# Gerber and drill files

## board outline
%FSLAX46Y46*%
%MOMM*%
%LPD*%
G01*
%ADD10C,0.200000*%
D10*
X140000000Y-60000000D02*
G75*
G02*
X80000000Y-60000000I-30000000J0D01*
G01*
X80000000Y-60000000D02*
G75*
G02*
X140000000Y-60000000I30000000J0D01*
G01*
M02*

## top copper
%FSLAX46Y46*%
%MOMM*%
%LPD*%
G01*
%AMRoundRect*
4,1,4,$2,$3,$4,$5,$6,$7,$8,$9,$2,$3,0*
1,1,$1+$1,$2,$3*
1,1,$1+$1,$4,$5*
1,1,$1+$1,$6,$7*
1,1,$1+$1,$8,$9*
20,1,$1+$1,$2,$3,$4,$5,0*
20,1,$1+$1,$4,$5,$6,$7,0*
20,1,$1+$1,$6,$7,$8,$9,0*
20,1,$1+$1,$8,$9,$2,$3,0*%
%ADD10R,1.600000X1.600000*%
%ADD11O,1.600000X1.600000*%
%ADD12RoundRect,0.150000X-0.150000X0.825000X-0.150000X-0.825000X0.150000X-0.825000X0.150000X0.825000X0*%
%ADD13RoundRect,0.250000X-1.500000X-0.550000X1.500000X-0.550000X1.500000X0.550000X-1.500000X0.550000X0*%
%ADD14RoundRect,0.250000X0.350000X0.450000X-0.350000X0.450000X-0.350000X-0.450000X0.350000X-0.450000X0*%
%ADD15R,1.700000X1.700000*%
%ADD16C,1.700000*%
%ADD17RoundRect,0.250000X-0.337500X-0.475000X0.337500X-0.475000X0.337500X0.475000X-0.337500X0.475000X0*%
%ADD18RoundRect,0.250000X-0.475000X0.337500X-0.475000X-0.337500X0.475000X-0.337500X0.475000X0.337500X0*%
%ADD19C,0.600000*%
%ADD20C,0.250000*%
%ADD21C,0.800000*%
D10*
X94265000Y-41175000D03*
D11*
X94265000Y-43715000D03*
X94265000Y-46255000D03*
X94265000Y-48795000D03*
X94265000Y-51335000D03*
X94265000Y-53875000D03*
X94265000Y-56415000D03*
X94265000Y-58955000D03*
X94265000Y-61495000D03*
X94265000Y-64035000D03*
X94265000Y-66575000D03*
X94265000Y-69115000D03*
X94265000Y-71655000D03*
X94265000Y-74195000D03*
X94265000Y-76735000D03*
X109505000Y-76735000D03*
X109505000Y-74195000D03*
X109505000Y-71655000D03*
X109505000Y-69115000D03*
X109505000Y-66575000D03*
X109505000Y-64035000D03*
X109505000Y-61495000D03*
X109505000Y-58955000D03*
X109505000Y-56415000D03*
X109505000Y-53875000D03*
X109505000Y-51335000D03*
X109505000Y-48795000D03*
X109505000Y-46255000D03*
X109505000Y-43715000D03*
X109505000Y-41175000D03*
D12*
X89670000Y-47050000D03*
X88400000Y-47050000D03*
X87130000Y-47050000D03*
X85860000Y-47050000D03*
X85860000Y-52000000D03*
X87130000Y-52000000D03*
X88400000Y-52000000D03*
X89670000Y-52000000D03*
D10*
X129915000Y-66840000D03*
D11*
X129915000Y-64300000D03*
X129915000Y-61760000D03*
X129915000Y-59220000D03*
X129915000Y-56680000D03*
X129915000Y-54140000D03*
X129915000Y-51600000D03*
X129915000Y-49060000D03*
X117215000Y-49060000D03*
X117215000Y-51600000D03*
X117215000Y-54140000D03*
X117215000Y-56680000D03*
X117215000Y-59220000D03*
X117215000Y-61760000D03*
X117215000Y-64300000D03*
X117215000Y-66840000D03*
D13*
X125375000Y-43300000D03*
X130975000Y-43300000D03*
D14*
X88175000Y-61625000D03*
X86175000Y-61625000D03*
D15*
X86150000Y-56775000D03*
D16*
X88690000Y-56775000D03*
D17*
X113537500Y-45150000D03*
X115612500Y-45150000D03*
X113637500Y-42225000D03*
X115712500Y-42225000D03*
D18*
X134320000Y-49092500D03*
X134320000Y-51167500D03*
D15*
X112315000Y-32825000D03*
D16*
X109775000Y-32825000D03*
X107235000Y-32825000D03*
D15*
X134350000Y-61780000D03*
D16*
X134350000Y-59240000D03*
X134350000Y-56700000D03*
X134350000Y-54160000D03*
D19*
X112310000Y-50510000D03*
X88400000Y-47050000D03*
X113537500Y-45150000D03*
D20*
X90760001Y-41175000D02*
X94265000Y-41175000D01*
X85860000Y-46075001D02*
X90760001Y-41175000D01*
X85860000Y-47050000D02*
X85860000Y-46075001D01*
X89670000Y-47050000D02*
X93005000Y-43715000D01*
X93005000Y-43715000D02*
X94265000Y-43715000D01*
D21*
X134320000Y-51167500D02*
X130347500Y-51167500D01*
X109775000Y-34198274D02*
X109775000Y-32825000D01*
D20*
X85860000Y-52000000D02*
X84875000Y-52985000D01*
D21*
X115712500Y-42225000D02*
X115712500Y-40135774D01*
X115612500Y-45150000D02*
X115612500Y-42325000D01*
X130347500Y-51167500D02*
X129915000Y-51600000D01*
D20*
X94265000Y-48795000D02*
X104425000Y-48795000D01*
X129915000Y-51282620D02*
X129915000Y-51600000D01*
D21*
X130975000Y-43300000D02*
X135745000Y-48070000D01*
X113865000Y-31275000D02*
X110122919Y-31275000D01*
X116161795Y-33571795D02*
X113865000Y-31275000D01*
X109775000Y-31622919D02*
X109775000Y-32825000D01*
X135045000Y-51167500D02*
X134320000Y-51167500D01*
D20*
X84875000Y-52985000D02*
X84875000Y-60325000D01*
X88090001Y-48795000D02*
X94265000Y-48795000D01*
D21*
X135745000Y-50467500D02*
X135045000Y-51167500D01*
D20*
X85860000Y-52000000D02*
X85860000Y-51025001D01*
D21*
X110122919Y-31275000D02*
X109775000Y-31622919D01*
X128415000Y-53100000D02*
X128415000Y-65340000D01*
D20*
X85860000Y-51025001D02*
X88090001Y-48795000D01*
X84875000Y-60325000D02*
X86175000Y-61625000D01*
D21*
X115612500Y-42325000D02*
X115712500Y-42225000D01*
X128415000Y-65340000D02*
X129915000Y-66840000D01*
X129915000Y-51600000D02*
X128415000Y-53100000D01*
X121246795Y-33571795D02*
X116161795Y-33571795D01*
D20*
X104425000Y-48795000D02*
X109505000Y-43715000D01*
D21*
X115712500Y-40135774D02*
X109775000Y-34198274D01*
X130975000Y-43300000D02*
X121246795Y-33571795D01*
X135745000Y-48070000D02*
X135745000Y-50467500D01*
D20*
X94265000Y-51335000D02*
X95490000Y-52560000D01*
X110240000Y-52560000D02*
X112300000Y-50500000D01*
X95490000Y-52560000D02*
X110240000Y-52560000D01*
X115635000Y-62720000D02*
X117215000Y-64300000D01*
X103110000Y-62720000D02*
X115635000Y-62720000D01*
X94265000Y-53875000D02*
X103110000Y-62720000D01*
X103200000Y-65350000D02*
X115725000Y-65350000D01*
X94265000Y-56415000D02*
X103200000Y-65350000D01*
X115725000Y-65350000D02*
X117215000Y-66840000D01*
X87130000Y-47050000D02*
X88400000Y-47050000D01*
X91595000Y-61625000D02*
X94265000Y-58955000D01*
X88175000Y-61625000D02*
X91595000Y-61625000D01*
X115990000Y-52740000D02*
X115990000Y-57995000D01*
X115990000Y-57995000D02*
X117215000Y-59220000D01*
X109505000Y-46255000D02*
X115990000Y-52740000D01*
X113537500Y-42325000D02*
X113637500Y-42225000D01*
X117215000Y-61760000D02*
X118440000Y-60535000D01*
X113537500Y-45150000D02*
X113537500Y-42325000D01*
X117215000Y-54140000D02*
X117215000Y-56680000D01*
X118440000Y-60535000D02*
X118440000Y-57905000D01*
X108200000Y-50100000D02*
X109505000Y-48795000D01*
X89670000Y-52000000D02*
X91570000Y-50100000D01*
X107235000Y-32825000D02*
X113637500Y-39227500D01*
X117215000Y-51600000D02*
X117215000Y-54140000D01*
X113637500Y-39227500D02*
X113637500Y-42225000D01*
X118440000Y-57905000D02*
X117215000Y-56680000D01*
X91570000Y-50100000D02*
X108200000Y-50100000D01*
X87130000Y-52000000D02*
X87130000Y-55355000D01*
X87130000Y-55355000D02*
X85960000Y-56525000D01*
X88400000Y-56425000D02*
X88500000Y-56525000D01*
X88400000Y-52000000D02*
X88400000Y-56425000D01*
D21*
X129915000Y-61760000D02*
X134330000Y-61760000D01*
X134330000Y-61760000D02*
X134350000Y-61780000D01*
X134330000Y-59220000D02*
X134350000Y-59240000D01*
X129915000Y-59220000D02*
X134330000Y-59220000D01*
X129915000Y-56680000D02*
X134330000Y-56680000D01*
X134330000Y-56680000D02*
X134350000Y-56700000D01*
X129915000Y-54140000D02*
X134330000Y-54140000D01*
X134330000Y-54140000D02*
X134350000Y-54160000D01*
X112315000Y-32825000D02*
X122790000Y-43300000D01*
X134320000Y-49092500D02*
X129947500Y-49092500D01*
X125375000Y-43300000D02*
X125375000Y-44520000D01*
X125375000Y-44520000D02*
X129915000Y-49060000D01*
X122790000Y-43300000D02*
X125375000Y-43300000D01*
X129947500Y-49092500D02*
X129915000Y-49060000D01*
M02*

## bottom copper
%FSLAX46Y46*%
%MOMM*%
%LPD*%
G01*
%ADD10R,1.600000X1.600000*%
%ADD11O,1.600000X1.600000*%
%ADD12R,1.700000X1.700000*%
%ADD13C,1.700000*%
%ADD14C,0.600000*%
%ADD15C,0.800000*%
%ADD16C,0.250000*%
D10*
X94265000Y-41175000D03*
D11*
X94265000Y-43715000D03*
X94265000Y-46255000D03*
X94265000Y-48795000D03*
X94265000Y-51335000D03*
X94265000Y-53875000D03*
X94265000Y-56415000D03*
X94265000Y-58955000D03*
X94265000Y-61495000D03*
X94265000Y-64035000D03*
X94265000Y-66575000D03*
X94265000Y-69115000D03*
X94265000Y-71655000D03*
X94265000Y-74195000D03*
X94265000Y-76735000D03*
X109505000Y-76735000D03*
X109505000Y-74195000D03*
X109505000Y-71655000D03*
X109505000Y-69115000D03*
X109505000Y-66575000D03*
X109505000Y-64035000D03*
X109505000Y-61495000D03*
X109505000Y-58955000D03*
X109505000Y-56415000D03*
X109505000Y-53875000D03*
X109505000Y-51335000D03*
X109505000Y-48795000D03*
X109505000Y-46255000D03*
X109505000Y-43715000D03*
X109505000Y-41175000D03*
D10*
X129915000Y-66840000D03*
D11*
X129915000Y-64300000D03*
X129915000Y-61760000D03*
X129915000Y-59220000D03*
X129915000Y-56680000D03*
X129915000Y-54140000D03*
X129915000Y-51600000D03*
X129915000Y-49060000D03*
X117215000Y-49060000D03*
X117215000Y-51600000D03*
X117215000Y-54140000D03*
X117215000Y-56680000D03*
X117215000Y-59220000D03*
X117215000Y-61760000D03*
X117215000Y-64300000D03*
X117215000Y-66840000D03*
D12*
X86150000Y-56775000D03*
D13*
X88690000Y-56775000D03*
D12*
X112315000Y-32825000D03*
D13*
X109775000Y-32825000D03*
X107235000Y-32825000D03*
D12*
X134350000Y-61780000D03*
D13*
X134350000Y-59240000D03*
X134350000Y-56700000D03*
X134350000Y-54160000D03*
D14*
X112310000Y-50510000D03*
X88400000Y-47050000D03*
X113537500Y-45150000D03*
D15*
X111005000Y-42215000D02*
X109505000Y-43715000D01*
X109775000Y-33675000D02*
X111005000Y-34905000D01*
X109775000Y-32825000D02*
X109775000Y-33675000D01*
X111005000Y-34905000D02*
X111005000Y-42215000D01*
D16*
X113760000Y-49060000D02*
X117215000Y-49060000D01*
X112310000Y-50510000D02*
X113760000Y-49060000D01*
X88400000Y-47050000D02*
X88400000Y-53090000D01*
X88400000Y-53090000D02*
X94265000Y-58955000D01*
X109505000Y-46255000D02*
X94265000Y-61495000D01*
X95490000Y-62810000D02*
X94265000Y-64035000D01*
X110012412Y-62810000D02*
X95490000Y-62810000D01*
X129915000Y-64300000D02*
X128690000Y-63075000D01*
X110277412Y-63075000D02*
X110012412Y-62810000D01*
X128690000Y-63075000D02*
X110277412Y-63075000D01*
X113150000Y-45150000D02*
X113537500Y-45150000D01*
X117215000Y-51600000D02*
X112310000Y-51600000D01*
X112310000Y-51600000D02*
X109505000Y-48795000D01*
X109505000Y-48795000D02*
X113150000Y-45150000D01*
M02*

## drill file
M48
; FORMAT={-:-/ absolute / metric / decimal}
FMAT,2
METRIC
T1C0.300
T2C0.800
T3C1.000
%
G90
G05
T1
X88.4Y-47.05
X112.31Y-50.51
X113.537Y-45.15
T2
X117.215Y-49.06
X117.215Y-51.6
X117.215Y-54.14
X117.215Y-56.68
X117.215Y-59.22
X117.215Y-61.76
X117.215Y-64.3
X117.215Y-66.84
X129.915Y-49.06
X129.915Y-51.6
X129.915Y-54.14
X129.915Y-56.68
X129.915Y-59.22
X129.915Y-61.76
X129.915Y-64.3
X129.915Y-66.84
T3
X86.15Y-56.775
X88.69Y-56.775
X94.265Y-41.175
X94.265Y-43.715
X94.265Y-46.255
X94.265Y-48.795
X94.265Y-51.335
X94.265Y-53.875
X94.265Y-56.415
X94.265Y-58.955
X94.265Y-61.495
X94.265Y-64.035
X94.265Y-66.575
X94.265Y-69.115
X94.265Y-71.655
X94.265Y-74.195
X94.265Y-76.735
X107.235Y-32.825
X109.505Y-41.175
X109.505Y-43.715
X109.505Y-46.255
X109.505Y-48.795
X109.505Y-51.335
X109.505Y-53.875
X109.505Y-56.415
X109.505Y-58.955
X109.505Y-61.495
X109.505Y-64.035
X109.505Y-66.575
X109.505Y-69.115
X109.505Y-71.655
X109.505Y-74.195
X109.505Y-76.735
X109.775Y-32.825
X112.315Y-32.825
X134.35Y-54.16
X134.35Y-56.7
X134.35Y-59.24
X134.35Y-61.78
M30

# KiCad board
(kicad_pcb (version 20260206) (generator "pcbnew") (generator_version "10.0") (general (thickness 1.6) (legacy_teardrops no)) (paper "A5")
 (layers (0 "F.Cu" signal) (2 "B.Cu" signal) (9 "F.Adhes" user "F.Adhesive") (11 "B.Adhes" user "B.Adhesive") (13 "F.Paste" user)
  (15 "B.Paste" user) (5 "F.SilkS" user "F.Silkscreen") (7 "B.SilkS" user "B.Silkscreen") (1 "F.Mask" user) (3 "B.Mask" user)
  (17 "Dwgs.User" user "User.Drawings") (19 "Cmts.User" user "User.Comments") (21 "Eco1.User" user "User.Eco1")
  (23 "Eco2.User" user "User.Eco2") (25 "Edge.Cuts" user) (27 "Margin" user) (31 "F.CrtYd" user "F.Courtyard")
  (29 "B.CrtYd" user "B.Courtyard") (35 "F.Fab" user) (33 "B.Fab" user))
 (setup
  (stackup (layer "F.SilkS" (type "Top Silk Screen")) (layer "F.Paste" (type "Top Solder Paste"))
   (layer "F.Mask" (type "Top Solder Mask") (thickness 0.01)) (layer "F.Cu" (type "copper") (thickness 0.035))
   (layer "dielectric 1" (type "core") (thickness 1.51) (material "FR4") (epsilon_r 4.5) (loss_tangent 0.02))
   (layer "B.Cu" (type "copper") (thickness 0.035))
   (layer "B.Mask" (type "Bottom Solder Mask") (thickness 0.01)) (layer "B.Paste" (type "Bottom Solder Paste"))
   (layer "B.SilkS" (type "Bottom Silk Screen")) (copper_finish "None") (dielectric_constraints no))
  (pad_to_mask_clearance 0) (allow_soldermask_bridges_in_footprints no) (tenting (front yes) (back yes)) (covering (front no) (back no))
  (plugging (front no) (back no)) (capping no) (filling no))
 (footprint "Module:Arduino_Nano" (layer "F.Cu") (at 94.265 41.175)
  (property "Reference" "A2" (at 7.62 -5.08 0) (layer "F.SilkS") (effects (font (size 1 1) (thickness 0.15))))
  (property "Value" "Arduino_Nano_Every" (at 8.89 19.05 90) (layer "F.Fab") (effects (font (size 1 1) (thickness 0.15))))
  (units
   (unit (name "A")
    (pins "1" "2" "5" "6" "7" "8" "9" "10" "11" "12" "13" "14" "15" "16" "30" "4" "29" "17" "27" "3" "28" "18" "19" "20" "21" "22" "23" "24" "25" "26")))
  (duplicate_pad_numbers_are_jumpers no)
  (pad "1" thru_hole rect (at 0 0) (size 1.6 1.6) (drill 1) (layers "*.Cu" "*.Mask") (remove_unused_layers no) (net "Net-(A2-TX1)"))
  (pad "2" thru_hole oval (at 0 2.54) (size 1.6 1.6) (drill 1) (layers "*.Cu" "*.Mask") (remove_unused_layers no) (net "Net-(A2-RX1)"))
  (pad "3" thru_hole oval (at 0 5.08) (size 1.6 1.6) (drill 1) (layers "*.Cu" "*.Mask") (remove_unused_layers no)
   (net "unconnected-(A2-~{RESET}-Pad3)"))
  (pad "4" thru_hole oval (at 0 7.62) (size 1.6 1.6) (drill 1) (layers "*.Cu" "*.Mask") (remove_unused_layers no) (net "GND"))
  (pad "5" thru_hole oval (at 0 10.16) (size 1.6 1.6) (drill 1) (layers "*.Cu" "*.Mask") (remove_unused_layers no) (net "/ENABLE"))
  (pad "6" thru_hole oval (at 0 12.7) (size 1.6 1.6) (drill 1) (layers "*.Cu" "*.Mask") (remove_unused_layers no) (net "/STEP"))
  (pad "7" thru_hole oval (at 0 15.24) (size 1.6 1.6) (drill 1) (layers "*.Cu" "*.Mask") (remove_unused_layers no) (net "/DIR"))
  (pad "8" thru_hole oval (at 0 17.78) (size 1.6 1.6) (drill 1) (layers "*.Cu" "*.Mask") (remove_unused_layers no) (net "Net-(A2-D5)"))
  (pad "9" thru_hole oval (at 0 20.32) (size 1.6 1.6) (drill 1) (layers "*.Cu" "*.Mask") (remove_unused_layers no) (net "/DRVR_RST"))
  (pad "10" thru_hole oval (at 0 22.86) (size 1.6 1.6) (drill 1) (layers "*.Cu" "*.Mask") (remove_unused_layers no) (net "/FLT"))
  (pad "11" thru_hole oval (at 0 25.4) (size 1.6 1.6) (drill 1) (layers "*.Cu" "*.Mask") (remove_unused_layers no)
   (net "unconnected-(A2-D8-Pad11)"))
  (pad "12" thru_hole oval (at 0 27.94) (size 1.6 1.6) (drill 1) (layers "*.Cu" "*.Mask") (remove_unused_layers no)
   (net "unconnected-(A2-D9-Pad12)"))
  (pad "13" thru_hole oval (at 0 30.48) (size 1.6 1.6) (drill 1) (layers "*.Cu" "*.Mask") (remove_unused_layers no)
   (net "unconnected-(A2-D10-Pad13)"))
  (pad "14" thru_hole oval (at 0 33.02) (size 1.6 1.6) (drill 1) (layers "*.Cu" "*.Mask") (remove_unused_layers no)
   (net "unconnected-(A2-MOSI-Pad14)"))
  (pad "15" thru_hole oval (at 0 35.56) (size 1.6 1.6) (drill 1) (layers "*.Cu" "*.Mask") (remove_unused_layers no)
   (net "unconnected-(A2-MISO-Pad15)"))
  (pad "16" thru_hole oval (at 15.24 35.56) (size 1.6 1.6) (drill 1) (layers "*.Cu" "*.Mask") (remove_unused_layers no)
   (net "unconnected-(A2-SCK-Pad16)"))
  (pad "17" thru_hole oval (at 15.24 33.02) (size 1.6 1.6) (drill 1) (layers "*.Cu" "*.Mask") (remove_unused_layers no)
   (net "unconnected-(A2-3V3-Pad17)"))
  (pad "18" thru_hole oval (at 15.24 30.48) (size 1.6 1.6) (drill 1) (layers "*.Cu" "*.Mask") (remove_unused_layers no)
   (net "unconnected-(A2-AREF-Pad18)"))
  (pad "19" thru_hole oval (at 15.24 27.94) (size 1.6 1.6) (drill 1) (layers "*.Cu" "*.Mask") (remove_unused_layers no)
   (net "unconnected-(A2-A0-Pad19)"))
  (pad "20" thru_hole oval (at 15.24 25.4) (size 1.6 1.6) (drill 1) (layers "*.Cu" "*.Mask") (remove_unused_layers no)
   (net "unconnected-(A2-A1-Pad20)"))
  (pad "21" thru_hole oval (at 15.24 22.86) (size 1.6 1.6) (drill 1) (layers "*.Cu" "*.Mask") (remove_unused_layers no)
   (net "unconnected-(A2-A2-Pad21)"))
  (pad "22" thru_hole oval (at 15.24 20.32) (size 1.6 1.6) (drill 1) (layers "*.Cu" "*.Mask") (remove_unused_layers no)
   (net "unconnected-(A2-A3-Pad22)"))
  (pad "23" thru_hole oval (at 15.24 17.78) (size 1.6 1.6) (drill 1) (layers "*.Cu" "*.Mask") (remove_unused_layers no)
   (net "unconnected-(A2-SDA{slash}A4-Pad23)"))
  (pad "24" thru_hole oval (at 15.24 15.24) (size 1.6 1.6) (drill 1) (layers "*.Cu" "*.Mask") (remove_unused_layers no)
   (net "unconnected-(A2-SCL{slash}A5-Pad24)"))
  (pad "25" thru_hole oval (at 15.24 12.7) (size 1.6 1.6) (drill 1) (layers "*.Cu" "*.Mask") (remove_unused_layers no)
   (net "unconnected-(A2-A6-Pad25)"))
  (pad "26" thru_hole oval (at 15.24 10.16) (size 1.6 1.6) (drill 1) (layers "*.Cu" "*.Mask") (remove_unused_layers no)
   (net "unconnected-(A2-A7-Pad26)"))
  (pad "27" thru_hole oval (at 15.24 7.62) (size 1.6 1.6) (drill 1) (layers "*.Cu" "*.Mask") (remove_unused_layers no) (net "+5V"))
  (pad "28" thru_hole oval (at 15.24 5.08) (size 1.6 1.6) (drill 1) (layers "*.Cu" "*.Mask") (remove_unused_layers no) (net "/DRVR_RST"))
  (pad "29" thru_hole oval (at 15.24 2.54) (size 1.6 1.6) (drill 1) (layers "*.Cu" "*.Mask") (remove_unused_layers no) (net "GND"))
  (pad "30" thru_hole oval (at 15.24 0) (size 1.6 1.6) (drill 1) (layers "*.Cu" "*.Mask") (remove_unused_layers no)
   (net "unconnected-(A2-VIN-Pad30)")))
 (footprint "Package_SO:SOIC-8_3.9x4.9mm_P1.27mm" (layer "F.Cu") (at 87.765 49.525 -90)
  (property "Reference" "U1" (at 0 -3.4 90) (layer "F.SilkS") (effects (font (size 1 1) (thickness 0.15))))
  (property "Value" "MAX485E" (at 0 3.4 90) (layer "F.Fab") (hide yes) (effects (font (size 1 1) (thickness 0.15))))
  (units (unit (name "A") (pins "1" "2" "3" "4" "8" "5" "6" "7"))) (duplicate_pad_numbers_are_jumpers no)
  (pad "1" smd roundrect (at -2.475 -1.905 270) (size 1.95 0.6) (layers "F.Cu" "F.Mask" "F.Paste") (roundrect_rratio 0.25)
   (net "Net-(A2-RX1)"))
  (pad "2" smd roundrect (at -2.475 -0.635 270) (size 1.95 0.6) (layers "F.Cu" "F.Mask" "F.Paste") (roundrect_rratio 0.25)
   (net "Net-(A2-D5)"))
  (pad "3" smd roundrect (at -2.475 0.635 270) (size 1.95 0.6) (layers "F.Cu" "F.Mask" "F.Paste") (roundrect_rratio 0.25)
   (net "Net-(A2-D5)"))
  (pad "4" smd roundrect (at -2.475 1.905 270) (size 1.95 0.6) (layers "F.Cu" "F.Mask" "F.Paste") (roundrect_rratio 0.25)
   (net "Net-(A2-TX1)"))
  (pad "5" smd roundrect (at 2.475 1.905 270) (size 1.95 0.6) (layers "F.Cu" "F.Mask" "F.Paste") (roundrect_rratio 0.25) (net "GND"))
  (pad "6" smd roundrect (at 2.475 0.635 270) (size 1.95 0.6) (layers "F.Cu" "F.Mask" "F.Paste") (roundrect_rratio 0.25)
   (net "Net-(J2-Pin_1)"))
  (pad "7" smd roundrect (at 2.475 -0.635 270) (size 1.95 0.6) (layers "F.Cu" "F.Mask" "F.Paste") (roundrect_rratio 0.25)
   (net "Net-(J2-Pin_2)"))
  (pad "8" smd roundrect (at 2.475 -1.905 270) (size 1.95 0.6) (layers "F.Cu" "F.Mask" "F.Paste") (roundrect_rratio 0.25) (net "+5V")))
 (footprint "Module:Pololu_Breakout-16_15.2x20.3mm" (layer "F.Cu") (at 129.915 66.84 180)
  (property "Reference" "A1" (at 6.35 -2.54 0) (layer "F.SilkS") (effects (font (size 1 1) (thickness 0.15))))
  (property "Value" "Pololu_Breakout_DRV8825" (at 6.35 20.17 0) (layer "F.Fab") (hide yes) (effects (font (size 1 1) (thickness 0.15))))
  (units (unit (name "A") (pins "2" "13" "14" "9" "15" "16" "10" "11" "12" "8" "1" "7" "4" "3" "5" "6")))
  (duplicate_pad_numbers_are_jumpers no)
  (pad "1" thru_hole rect (at 0 0 180) (size 1.6 1.6) (drill 0.8) (layers "*.Cu" "*.Mask") (remove_unused_layers no) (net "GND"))
  (pad "2" thru_hole oval (at 0 2.54 180) (size 1.6 1.6) (drill 0.8) (layers "*.Cu" "*.Mask") (remove_unused_layers no) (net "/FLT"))
  (pad "3" thru_hole oval (at 0 5.08 180) (size 1.6 1.6) (drill 0.8) (layers "*.Cu" "*.Mask") (remove_unused_layers no) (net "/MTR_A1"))
  (pad "4" thru_hole oval (at 0 7.62 180) (size 1.6 1.6) (drill 0.8) (layers "*.Cu" "*.Mask") (remove_unused_layers no) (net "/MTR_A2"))
  (pad "5" thru_hole oval (at 0 10.16 180) (size 1.6 1.6) (drill 0.8) (layers "*.Cu" "*.Mask") (remove_unused_layers no) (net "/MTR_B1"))
  (pad "6" thru_hole oval (at 0 12.7 180) (size 1.6 1.6) (drill 0.8) (layers "*.Cu" "*.Mask") (remove_unused_layers no) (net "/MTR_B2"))
  (pad "7" thru_hole oval (at 0 15.24 180) (size 1.6 1.6) (drill 0.8) (layers "*.Cu" "*.Mask") (remove_unused_layers no) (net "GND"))
  (pad "8" thru_hole oval (at 0 17.78 180) (size 1.6 1.6) (drill 0.8) (layers "*.Cu" "*.Mask") (remove_unused_layers no) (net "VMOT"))
  (pad "9" thru_hole oval (at 12.7 17.78 180) (size 1.6 1.6) (drill 0.8) (layers "*.Cu" "*.Mask") (remove_unused_layers no) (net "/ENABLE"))
  (pad "10" thru_hole oval (at 12.7 15.24 180) (size 1.6 1.6) (drill 0.8) (layers "*.Cu" "*.Mask") (remove_unused_layers no) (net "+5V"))
  (pad "11" thru_hole oval (at 12.7 12.7 180) (size 1.6 1.6) (drill 0.8) (layers "*.Cu" "*.Mask") (remove_unused_layers no) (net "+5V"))
  (pad "12" thru_hole oval (at 12.7 10.16 180) (size 1.6 1.6) (drill 0.8) (layers "*.Cu" "*.Mask") (remove_unused_layers no) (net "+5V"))
  (pad "13" thru_hole oval (at 12.7 7.62 180) (size 1.6 1.6) (drill 0.8) (layers "*.Cu" "*.Mask") (remove_unused_layers no)
   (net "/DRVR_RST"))
  (pad "14" thru_hole oval (at 12.7 5.08 180) (size 1.6 1.6) (drill 0.8) (layers "*.Cu" "*.Mask") (remove_unused_layers no) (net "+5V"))
  (pad "15" thru_hole oval (at 12.7 2.54 180) (size 1.6 1.6) (drill 0.8) (layers "*.Cu" "*.Mask") (remove_unused_layers no) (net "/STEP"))
  (pad "16" thru_hole oval (at 12.7 0 180) (size 1.6 1.6) (drill 0.8) (layers "*.Cu" "*.Mask") (remove_unused_layers no) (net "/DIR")))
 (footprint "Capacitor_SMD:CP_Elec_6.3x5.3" (layer "F.Cu") (at 128.175 43.3)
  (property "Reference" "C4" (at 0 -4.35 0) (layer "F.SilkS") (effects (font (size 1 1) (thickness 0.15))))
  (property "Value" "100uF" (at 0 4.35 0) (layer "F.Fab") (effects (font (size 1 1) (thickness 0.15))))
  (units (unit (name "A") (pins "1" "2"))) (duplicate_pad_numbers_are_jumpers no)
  (pad "1" smd roundrect (at -2.8 0) (size 3.5 1.6) (layers "F.Cu" "F.Mask" "F.Paste") (roundrect_rratio 0.15625) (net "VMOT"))
  (pad "2" smd roundrect (at 2.8 0) (size 3.5 1.6) (layers "F.Cu" "F.Mask" "F.Paste") (roundrect_rratio 0.15625) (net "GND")))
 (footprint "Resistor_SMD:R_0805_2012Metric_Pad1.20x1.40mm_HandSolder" (layer "F.Cu") (at 87.175 61.625 180)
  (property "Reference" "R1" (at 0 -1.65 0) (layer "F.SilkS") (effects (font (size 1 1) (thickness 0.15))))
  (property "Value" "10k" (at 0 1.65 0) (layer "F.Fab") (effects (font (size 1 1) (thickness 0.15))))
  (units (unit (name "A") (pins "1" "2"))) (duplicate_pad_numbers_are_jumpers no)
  (pad "1" smd roundrect (at -1 0 180) (size 1.2 1.4) (layers "F.Cu" "F.Mask" "F.Paste") (roundrect_rratio 0.208333) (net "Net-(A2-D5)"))
  (pad "2" smd roundrect (at 1 0 180) (size 1.2 1.4) (layers "F.Cu" "F.Mask" "F.Paste") (roundrect_rratio 0.208333) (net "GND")))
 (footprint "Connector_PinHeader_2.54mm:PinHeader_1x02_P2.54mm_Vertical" (layer "F.Cu") (at 86.15 56.775 90)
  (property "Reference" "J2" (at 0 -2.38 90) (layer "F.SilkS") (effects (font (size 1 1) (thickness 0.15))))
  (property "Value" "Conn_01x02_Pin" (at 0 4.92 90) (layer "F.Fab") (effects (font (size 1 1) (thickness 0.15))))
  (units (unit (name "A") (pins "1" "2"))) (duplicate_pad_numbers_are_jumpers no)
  (pad "1" thru_hole rect (at 0 0 90) (size 1.7 1.7) (drill 1) (layers "*.Cu" "*.Mask") (remove_unused_layers no) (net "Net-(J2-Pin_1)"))
  (pad "2" thru_hole circle (at 0 2.54 90) (size 1.7 1.7) (drill 1) (layers "*.Cu" "*.Mask") (remove_unused_layers no)
   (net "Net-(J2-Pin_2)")))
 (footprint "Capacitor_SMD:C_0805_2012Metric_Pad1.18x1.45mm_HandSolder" (layer "F.Cu") (at 114.575 45.15)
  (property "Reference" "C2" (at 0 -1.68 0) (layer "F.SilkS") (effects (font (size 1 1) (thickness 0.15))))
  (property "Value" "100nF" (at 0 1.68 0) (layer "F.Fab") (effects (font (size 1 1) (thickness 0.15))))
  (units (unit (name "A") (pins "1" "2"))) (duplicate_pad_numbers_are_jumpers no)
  (pad "1" smd roundrect (at -1.0375 0) (size 1.175 1.45) (layers "F.Cu" "F.Mask" "F.Paste") (roundrect_rratio 0.212766) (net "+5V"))
  (pad "2" smd roundrect (at 1.0375 0) (size 1.175 1.45) (layers "F.Cu" "F.Mask" "F.Paste") (roundrect_rratio 0.212766) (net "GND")))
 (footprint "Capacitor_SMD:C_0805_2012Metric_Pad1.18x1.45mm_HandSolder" (layer "F.Cu") (at 114.675 42.225)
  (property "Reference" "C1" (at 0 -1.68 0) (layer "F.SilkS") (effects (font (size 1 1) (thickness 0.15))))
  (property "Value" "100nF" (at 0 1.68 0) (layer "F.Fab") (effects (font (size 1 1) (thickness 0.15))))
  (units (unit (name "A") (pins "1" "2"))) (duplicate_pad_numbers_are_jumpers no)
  (pad "1" smd roundrect (at -1.0375 0) (size 1.175 1.45) (layers "F.Cu" "F.Mask" "F.Paste") (roundrect_rratio 0.212766) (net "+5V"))
  (pad "2" smd roundrect (at 1.0375 0) (size 1.175 1.45) (layers "F.Cu" "F.Mask" "F.Paste") (roundrect_rratio 0.212766) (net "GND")))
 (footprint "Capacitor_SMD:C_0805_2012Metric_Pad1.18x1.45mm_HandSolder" (layer "F.Cu") (at 134.32 50.13 -90)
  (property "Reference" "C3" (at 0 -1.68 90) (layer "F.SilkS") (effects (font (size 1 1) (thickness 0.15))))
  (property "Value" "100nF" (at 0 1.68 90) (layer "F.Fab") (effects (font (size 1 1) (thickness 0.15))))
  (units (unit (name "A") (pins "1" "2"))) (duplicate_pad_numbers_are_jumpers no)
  (pad "1" smd roundrect (at -1.0375 0 270) (size 1.175 1.45) (layers "F.Cu" "F.Mask" "F.Paste") (roundrect_rratio 0.212766) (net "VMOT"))
  (pad "2" smd roundrect (at 1.0375 0 270) (size 1.175 1.45) (layers "F.Cu" "F.Mask" "F.Paste") (roundrect_rratio 0.212766) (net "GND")))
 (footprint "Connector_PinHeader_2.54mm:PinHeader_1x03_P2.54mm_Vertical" (layer "F.Cu") (at 112.315 32.825 -90)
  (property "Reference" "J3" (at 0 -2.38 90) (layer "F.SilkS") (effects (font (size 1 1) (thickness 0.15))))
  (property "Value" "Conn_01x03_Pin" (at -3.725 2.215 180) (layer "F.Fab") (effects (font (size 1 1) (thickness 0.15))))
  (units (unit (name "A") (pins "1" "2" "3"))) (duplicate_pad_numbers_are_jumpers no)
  (pad "1" thru_hole rect (at 0 0 270) (size 1.7 1.7) (drill 1) (layers "*.Cu" "*.Mask") (remove_unused_layers no) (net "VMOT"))
  (pad "2" thru_hole circle (at 0 2.54 270) (size 1.7 1.7) (drill 1) (layers "*.Cu" "*.Mask") (remove_unused_layers no) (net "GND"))
  (pad "3" thru_hole circle (at 0 5.08 270) (size 1.7 1.7) (drill 1) (layers "*.Cu" "*.Mask") (remove_unused_layers no) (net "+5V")))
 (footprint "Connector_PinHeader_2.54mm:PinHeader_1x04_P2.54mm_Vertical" (layer "B.Cu") (at 134.35 61.78)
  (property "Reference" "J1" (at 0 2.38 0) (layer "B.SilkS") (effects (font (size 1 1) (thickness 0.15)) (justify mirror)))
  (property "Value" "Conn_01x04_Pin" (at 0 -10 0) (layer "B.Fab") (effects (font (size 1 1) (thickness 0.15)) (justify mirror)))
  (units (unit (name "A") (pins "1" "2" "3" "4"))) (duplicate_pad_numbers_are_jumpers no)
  (pad "1" thru_hole rect (at 0 0) (size 1.7 1.7) (drill 1) (layers "*.Cu" "*.Mask") (remove_unused_layers no) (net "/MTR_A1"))
  (pad "2" thru_hole circle (at 0 -2.54) (size 1.7 1.7) (drill 1) (layers "*.Cu" "*.Mask") (remove_unused_layers no) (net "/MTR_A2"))
  (pad "3" thru_hole circle (at 0 -5.08) (size 1.7 1.7) (drill 1) (layers "*.Cu" "*.Mask") (remove_unused_layers no) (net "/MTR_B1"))
  (pad "4" thru_hole circle (at 0 -7.62) (size 1.7 1.7) (drill 1) (layers "*.Cu" "*.Mask") (remove_unused_layers no) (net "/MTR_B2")))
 (gr_circle (center 110 60) (end 140 60) (stroke (width 0.2) (type solid)) (fill no) (layer "Edge.Cuts"))
 (segment (start 90.760001 41.175) (end 94.265 41.175) (width 0.25) (layer "F.Cu") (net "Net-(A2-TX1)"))
 (segment (start 85.86 46.075001) (end 90.760001 41.175) (width 0.25) (layer "F.Cu") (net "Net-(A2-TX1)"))
 (segment (start 85.86 47.05) (end 85.86 46.075001) (width 0.25) (layer "F.Cu") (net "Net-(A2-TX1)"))
 (segment (start 89.67 47.05) (end 93.005 43.715) (width 0.25) (layer "F.Cu") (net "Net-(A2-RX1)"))
 (segment (start 93.005 43.715) (end 94.265 43.715) (width 0.25) (layer "F.Cu") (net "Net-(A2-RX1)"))
 (segment (start 134.32 51.1675) (end 130.3475 51.1675) (width 0.8) (layer "F.Cu") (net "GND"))
 (segment (start 109.775 34.198274) (end 109.775 32.825) (width 0.8) (layer "F.Cu") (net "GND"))
 (segment (start 85.86 52) (end 84.875 52.985) (width 0.25) (layer "F.Cu") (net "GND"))
 (segment (start 115.7125 42.225) (end 115.7125 40.135774) (width 0.8) (layer "F.Cu") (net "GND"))
 (segment (start 115.6125 45.15) (end 115.6125 42.325) (width 0.8) (layer "F.Cu") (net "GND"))
 (segment (start 130.3475 51.1675) (end 129.915 51.6) (width 0.8) (layer "F.Cu") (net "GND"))
 (segment (start 94.265 48.795) (end 104.425 48.795) (width 0.25) (layer "F.Cu") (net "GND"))
 (segment (start 129.915 51.28262) (end 129.915 51.6) (width 0.25) (layer "F.Cu") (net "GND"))
 (segment (start 130.975 43.3) (end 135.745 48.07) (width 0.8) (layer "F.Cu") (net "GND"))
 (segment (start 113.865 31.275) (end 110.122919 31.275) (width 0.8) (layer "F.Cu") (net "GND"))
 (segment (start 116.161795 33.571795) (end 113.865 31.275) (width 0.8) (layer "F.Cu") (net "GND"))
 (segment (start 109.775 31.622919) (end 109.775 32.825) (width 0.8) (layer "F.Cu") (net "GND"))
 (segment (start 135.045 51.1675) (end 134.32 51.1675) (width 0.8) (layer "F.Cu") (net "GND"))
 (segment (start 84.875 52.985) (end 84.875 60.325) (width 0.25) (layer "F.Cu") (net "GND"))
 (segment (start 88.090001 48.795) (end 94.265 48.795) (width 0.25) (layer "F.Cu") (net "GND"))
 (segment (start 135.745 50.4675) (end 135.045 51.1675) (width 0.8) (layer "F.Cu") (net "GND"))
 (segment (start 85.86 52) (end 85.86 51.025001) (width 0.25) (layer "F.Cu") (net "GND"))
 (segment (start 110.122919 31.275) (end 109.775 31.622919) (width 0.8) (layer "F.Cu") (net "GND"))
 (segment (start 128.415 53.1) (end 128.415 65.34) (width 0.8) (layer "F.Cu") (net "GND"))
 (segment (start 85.86 51.025001) (end 88.090001 48.795) (width 0.25) (layer "F.Cu") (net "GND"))
 (segment (start 84.875 60.325) (end 86.175 61.625) (width 0.25) (layer "F.Cu") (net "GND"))
 (segment (start 115.6125 42.325) (end 115.7125 42.225) (width 0.8) (layer "F.Cu") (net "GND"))
 (segment (start 128.415 65.34) (end 129.915 66.84) (width 0.8) (layer "F.Cu") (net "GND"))
 (segment (start 129.915 51.6) (end 128.415 53.1) (width 0.8) (layer "F.Cu") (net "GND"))
 (segment (start 121.246795 33.571795) (end 116.161795 33.571795) (width 0.8) (layer "F.Cu") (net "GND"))
 (segment (start 104.425 48.795) (end 109.505 43.715) (width 0.25) (layer "F.Cu") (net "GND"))
 (segment (start 115.7125 40.135774) (end 109.775 34.198274) (width 0.8) (layer "F.Cu") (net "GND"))
 (segment (start 130.975 43.3) (end 121.246795 33.571795) (width 0.8) (layer "F.Cu") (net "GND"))
 (segment (start 135.745 48.07) (end 135.745 50.4675) (width 0.8) (layer "F.Cu") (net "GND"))
 (segment (start 111.005 42.215) (end 109.505 43.715) (width 0.8) (layer "B.Cu") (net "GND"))
 (segment (start 109.775 33.675) (end 111.005 34.905) (width 0.8) (layer "B.Cu") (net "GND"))
 (segment (start 109.775 32.825) (end 109.775 33.675) (width 0.8) (layer "B.Cu") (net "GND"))
 (segment (start 111.005 34.905) (end 111.005 42.215) (width 0.8) (layer "B.Cu") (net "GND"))
 (segment (start 94.265 51.335) (end 95.49 52.56) (width 0.25) (layer "F.Cu") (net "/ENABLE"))
 (segment (start 110.24 52.56) (end 112.3 50.5) (width 0.25) (layer "F.Cu") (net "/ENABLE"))
 (segment (start 95.49 52.56) (end 110.24 52.56) (width 0.25) (layer "F.Cu") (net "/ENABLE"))
 (via (at 112.31 50.51) (size 0.6) (drill 0.3) (layers "F.Cu" "B.Cu") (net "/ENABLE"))
 (segment (start 113.76 49.06) (end 117.215 49.06) (width 0.25) (layer "B.Cu") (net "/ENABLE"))
 (segment (start 112.31 50.51) (end 113.76 49.06) (width 0.25) (layer "B.Cu") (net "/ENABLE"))
 (segment (start 115.635 62.72) (end 117.215 64.3) (width 0.25) (layer "F.Cu") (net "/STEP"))
 (segment (start 103.11 62.72) (end 115.635 62.72) (width 0.25) (layer "F.Cu") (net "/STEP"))
 (segment (start 94.265 53.875) (end 103.11 62.72) (width 0.25) (layer "F.Cu") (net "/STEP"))
 (segment (start 103.2 65.35) (end 115.725 65.35) (width 0.25) (layer "F.Cu") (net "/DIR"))
 (segment (start 94.265 56.415) (end 103.2 65.35) (width 0.25) (layer "F.Cu") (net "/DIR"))
 (segment (start 115.725 65.35) (end 117.215 66.84) (width 0.25) (layer "F.Cu") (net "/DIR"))
 (segment (start 87.13 47.05) (end 88.4 47.05) (width 0.25) (layer "F.Cu") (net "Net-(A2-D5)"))
 (segment (start 91.595 61.625) (end 94.265 58.955) (width 0.25) (layer "F.Cu") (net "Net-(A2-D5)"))
 (segment (start 88.175 61.625) (end 91.595 61.625) (width 0.25) (layer "F.Cu") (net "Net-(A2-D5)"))
 (via (at 88.4 47.05) (size 0.6) (drill 0.3) (layers "F.Cu" "B.Cu") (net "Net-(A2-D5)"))
 (segment (start 88.4 47.05) (end 88.4 53.09) (width 0.25) (layer "B.Cu") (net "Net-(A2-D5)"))
 (segment (start 88.4 53.09) (end 94.265 58.955) (width 0.25) (layer "B.Cu") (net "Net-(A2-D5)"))
 (segment (start 115.99 52.74) (end 115.99 57.995) (width 0.25) (layer "F.Cu") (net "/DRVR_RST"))
 (segment (start 115.99 57.995) (end 117.215 59.22) (width 0.25) (layer "F.Cu") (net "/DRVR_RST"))
 (segment (start 109.505 46.255) (end 115.99 52.74) (width 0.25) (layer "F.Cu") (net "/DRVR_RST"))
 (segment (start 109.505 46.255) (end 94.265 61.495) (width 0.25) (layer "B.Cu") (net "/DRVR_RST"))
 (segment (start 95.49 62.81) (end 94.265 64.035) (width 0.25) (layer "B.Cu") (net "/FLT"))
 (segment (start 110.012412 62.81) (end 95.49 62.81) (width 0.25) (layer "B.Cu") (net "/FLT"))
 (segment (start 129.915 64.3) (end 128.69 63.075) (width 0.25) (layer "B.Cu") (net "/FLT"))
 (segment (start 110.277412 63.075) (end 110.012412 62.81) (width 0.25) (layer "B.Cu") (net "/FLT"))
 (segment (start 128.69 63.075) (end 110.277412 63.075) (width 0.25) (layer "B.Cu") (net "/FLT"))
 (segment (start 113.5375 42.325) (end 113.6375 42.225) (width 0.25) (layer "F.Cu") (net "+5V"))
 (segment (start 117.215 61.76) (end 118.44 60.535) (width 0.25) (layer "F.Cu") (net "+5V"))
 (segment (start 113.5375 45.15) (end 113.5375 42.325) (width 0.25) (layer "F.Cu") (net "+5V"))
 (segment (start 117.215 54.14) (end 117.215 56.68) (width 0.25) (layer "F.Cu") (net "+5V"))
 (segment (start 118.44 60.535) (end 118.44 57.905) (width 0.25) (layer "F.Cu") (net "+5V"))
 (segment (start 108.2 50.1) (end 109.505 48.795) (width 0.25) (layer "F.Cu") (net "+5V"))
 (segment (start 89.67 52) (end 91.57 50.1) (width 0.25) (layer "F.Cu") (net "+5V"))
 (segment (start 107.235 32.825) (end 113.6375 39.2275) (width 0.25) (layer "F.Cu") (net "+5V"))
 (segment (start 117.215 51.6) (end 117.215 54.14) (width 0.25) (layer "F.Cu") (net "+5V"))
 (segment (start 113.6375 39.2275) (end 113.6375 42.225) (width 0.25) (layer "F.Cu") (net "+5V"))
 (segment (start 118.44 57.905) (end 117.215 56.68) (width 0.25) (layer "F.Cu") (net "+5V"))
 (segment (start 91.57 50.1) (end 108.2 50.1) (width 0.25) (layer "F.Cu") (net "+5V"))
 (via (at 113.5375 45.15) (size 0.6) (drill 0.3) (layers "F.Cu" "B.Cu") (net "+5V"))
 (segment (start 113.15 45.15) (end 113.5375 45.15) (width 0.25) (layer "B.Cu") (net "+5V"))
 (segment (start 117.215 51.6) (end 112.31 51.6) (width 0.25) (layer "B.Cu") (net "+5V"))
 (segment (start 112.31 51.6) (end 109.505 48.795) (width 0.25) (layer "B.Cu") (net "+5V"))
 (segment (start 109.505 48.795) (end 113.15 45.15) (width 0.25) (layer "B.Cu") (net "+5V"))
 (segment (start 87.13 52) (end 87.13 55.355) (width 0.25) (layer "F.Cu") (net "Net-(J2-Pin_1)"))
 (segment (start 87.13 55.355) (end 85.96 56.525) (width 0.25) (layer "F.Cu") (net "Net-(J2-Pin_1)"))
 (segment (start 88.4 56.425) (end 88.5 56.525) (width 0.25) (layer "F.Cu") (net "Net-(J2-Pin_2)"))
 (segment (start 88.4 52) (end 88.4 56.425) (width 0.25) (layer "F.Cu") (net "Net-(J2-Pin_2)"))
 (segment (start 129.915 61.76) (end 134.33 61.76) (width 0.8) (layer "F.Cu") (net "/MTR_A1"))
 (segment (start 134.33 61.76) (end 134.35 61.78) (width 0.8) (layer "F.Cu") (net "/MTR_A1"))
 (segment (start 134.33 59.22) (end 134.35 59.24) (width 0.8) (layer "F.Cu") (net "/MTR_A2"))
 (segment (start 129.915 59.22) (end 134.33 59.22) (width 0.8) (layer "F.Cu") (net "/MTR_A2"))
 (segment (start 129.915 56.68) (end 134.33 56.68) (width 0.8) (layer "F.Cu") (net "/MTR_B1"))
 (segment (start 134.33 56.68) (end 134.35 56.7) (width 0.8) (layer "F.Cu") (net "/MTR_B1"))
 (segment (start 129.915 54.14) (end 134.33 54.14) (width 0.8) (layer "F.Cu") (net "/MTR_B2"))
 (segment (start 134.33 54.14) (end 134.35 54.16) (width 0.8) (layer "F.Cu") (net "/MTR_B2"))
 (segment (start 112.315 32.825) (end 122.79 43.3) (width 0.8) (layer "F.Cu") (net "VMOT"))
 (segment (start 134.32 49.0925) (end 129.9475 49.0925) (width 0.8) (layer "F.Cu") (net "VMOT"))
 (segment (start 125.375 43.3) (end 125.375 44.52) (width 0.8) (layer "F.Cu") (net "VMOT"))
 (segment (start 125.375 44.52) (end 129.915 49.06) (width 0.8) (layer "F.Cu") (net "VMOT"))
 (segment (start 122.79 43.3) (end 125.375 43.3) (width 0.8) (layer "F.Cu") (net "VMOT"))
 (segment (start 129.9475 49.0925) (end 129.915 49.06) (width 0.8) (layer "F.Cu") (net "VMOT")))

